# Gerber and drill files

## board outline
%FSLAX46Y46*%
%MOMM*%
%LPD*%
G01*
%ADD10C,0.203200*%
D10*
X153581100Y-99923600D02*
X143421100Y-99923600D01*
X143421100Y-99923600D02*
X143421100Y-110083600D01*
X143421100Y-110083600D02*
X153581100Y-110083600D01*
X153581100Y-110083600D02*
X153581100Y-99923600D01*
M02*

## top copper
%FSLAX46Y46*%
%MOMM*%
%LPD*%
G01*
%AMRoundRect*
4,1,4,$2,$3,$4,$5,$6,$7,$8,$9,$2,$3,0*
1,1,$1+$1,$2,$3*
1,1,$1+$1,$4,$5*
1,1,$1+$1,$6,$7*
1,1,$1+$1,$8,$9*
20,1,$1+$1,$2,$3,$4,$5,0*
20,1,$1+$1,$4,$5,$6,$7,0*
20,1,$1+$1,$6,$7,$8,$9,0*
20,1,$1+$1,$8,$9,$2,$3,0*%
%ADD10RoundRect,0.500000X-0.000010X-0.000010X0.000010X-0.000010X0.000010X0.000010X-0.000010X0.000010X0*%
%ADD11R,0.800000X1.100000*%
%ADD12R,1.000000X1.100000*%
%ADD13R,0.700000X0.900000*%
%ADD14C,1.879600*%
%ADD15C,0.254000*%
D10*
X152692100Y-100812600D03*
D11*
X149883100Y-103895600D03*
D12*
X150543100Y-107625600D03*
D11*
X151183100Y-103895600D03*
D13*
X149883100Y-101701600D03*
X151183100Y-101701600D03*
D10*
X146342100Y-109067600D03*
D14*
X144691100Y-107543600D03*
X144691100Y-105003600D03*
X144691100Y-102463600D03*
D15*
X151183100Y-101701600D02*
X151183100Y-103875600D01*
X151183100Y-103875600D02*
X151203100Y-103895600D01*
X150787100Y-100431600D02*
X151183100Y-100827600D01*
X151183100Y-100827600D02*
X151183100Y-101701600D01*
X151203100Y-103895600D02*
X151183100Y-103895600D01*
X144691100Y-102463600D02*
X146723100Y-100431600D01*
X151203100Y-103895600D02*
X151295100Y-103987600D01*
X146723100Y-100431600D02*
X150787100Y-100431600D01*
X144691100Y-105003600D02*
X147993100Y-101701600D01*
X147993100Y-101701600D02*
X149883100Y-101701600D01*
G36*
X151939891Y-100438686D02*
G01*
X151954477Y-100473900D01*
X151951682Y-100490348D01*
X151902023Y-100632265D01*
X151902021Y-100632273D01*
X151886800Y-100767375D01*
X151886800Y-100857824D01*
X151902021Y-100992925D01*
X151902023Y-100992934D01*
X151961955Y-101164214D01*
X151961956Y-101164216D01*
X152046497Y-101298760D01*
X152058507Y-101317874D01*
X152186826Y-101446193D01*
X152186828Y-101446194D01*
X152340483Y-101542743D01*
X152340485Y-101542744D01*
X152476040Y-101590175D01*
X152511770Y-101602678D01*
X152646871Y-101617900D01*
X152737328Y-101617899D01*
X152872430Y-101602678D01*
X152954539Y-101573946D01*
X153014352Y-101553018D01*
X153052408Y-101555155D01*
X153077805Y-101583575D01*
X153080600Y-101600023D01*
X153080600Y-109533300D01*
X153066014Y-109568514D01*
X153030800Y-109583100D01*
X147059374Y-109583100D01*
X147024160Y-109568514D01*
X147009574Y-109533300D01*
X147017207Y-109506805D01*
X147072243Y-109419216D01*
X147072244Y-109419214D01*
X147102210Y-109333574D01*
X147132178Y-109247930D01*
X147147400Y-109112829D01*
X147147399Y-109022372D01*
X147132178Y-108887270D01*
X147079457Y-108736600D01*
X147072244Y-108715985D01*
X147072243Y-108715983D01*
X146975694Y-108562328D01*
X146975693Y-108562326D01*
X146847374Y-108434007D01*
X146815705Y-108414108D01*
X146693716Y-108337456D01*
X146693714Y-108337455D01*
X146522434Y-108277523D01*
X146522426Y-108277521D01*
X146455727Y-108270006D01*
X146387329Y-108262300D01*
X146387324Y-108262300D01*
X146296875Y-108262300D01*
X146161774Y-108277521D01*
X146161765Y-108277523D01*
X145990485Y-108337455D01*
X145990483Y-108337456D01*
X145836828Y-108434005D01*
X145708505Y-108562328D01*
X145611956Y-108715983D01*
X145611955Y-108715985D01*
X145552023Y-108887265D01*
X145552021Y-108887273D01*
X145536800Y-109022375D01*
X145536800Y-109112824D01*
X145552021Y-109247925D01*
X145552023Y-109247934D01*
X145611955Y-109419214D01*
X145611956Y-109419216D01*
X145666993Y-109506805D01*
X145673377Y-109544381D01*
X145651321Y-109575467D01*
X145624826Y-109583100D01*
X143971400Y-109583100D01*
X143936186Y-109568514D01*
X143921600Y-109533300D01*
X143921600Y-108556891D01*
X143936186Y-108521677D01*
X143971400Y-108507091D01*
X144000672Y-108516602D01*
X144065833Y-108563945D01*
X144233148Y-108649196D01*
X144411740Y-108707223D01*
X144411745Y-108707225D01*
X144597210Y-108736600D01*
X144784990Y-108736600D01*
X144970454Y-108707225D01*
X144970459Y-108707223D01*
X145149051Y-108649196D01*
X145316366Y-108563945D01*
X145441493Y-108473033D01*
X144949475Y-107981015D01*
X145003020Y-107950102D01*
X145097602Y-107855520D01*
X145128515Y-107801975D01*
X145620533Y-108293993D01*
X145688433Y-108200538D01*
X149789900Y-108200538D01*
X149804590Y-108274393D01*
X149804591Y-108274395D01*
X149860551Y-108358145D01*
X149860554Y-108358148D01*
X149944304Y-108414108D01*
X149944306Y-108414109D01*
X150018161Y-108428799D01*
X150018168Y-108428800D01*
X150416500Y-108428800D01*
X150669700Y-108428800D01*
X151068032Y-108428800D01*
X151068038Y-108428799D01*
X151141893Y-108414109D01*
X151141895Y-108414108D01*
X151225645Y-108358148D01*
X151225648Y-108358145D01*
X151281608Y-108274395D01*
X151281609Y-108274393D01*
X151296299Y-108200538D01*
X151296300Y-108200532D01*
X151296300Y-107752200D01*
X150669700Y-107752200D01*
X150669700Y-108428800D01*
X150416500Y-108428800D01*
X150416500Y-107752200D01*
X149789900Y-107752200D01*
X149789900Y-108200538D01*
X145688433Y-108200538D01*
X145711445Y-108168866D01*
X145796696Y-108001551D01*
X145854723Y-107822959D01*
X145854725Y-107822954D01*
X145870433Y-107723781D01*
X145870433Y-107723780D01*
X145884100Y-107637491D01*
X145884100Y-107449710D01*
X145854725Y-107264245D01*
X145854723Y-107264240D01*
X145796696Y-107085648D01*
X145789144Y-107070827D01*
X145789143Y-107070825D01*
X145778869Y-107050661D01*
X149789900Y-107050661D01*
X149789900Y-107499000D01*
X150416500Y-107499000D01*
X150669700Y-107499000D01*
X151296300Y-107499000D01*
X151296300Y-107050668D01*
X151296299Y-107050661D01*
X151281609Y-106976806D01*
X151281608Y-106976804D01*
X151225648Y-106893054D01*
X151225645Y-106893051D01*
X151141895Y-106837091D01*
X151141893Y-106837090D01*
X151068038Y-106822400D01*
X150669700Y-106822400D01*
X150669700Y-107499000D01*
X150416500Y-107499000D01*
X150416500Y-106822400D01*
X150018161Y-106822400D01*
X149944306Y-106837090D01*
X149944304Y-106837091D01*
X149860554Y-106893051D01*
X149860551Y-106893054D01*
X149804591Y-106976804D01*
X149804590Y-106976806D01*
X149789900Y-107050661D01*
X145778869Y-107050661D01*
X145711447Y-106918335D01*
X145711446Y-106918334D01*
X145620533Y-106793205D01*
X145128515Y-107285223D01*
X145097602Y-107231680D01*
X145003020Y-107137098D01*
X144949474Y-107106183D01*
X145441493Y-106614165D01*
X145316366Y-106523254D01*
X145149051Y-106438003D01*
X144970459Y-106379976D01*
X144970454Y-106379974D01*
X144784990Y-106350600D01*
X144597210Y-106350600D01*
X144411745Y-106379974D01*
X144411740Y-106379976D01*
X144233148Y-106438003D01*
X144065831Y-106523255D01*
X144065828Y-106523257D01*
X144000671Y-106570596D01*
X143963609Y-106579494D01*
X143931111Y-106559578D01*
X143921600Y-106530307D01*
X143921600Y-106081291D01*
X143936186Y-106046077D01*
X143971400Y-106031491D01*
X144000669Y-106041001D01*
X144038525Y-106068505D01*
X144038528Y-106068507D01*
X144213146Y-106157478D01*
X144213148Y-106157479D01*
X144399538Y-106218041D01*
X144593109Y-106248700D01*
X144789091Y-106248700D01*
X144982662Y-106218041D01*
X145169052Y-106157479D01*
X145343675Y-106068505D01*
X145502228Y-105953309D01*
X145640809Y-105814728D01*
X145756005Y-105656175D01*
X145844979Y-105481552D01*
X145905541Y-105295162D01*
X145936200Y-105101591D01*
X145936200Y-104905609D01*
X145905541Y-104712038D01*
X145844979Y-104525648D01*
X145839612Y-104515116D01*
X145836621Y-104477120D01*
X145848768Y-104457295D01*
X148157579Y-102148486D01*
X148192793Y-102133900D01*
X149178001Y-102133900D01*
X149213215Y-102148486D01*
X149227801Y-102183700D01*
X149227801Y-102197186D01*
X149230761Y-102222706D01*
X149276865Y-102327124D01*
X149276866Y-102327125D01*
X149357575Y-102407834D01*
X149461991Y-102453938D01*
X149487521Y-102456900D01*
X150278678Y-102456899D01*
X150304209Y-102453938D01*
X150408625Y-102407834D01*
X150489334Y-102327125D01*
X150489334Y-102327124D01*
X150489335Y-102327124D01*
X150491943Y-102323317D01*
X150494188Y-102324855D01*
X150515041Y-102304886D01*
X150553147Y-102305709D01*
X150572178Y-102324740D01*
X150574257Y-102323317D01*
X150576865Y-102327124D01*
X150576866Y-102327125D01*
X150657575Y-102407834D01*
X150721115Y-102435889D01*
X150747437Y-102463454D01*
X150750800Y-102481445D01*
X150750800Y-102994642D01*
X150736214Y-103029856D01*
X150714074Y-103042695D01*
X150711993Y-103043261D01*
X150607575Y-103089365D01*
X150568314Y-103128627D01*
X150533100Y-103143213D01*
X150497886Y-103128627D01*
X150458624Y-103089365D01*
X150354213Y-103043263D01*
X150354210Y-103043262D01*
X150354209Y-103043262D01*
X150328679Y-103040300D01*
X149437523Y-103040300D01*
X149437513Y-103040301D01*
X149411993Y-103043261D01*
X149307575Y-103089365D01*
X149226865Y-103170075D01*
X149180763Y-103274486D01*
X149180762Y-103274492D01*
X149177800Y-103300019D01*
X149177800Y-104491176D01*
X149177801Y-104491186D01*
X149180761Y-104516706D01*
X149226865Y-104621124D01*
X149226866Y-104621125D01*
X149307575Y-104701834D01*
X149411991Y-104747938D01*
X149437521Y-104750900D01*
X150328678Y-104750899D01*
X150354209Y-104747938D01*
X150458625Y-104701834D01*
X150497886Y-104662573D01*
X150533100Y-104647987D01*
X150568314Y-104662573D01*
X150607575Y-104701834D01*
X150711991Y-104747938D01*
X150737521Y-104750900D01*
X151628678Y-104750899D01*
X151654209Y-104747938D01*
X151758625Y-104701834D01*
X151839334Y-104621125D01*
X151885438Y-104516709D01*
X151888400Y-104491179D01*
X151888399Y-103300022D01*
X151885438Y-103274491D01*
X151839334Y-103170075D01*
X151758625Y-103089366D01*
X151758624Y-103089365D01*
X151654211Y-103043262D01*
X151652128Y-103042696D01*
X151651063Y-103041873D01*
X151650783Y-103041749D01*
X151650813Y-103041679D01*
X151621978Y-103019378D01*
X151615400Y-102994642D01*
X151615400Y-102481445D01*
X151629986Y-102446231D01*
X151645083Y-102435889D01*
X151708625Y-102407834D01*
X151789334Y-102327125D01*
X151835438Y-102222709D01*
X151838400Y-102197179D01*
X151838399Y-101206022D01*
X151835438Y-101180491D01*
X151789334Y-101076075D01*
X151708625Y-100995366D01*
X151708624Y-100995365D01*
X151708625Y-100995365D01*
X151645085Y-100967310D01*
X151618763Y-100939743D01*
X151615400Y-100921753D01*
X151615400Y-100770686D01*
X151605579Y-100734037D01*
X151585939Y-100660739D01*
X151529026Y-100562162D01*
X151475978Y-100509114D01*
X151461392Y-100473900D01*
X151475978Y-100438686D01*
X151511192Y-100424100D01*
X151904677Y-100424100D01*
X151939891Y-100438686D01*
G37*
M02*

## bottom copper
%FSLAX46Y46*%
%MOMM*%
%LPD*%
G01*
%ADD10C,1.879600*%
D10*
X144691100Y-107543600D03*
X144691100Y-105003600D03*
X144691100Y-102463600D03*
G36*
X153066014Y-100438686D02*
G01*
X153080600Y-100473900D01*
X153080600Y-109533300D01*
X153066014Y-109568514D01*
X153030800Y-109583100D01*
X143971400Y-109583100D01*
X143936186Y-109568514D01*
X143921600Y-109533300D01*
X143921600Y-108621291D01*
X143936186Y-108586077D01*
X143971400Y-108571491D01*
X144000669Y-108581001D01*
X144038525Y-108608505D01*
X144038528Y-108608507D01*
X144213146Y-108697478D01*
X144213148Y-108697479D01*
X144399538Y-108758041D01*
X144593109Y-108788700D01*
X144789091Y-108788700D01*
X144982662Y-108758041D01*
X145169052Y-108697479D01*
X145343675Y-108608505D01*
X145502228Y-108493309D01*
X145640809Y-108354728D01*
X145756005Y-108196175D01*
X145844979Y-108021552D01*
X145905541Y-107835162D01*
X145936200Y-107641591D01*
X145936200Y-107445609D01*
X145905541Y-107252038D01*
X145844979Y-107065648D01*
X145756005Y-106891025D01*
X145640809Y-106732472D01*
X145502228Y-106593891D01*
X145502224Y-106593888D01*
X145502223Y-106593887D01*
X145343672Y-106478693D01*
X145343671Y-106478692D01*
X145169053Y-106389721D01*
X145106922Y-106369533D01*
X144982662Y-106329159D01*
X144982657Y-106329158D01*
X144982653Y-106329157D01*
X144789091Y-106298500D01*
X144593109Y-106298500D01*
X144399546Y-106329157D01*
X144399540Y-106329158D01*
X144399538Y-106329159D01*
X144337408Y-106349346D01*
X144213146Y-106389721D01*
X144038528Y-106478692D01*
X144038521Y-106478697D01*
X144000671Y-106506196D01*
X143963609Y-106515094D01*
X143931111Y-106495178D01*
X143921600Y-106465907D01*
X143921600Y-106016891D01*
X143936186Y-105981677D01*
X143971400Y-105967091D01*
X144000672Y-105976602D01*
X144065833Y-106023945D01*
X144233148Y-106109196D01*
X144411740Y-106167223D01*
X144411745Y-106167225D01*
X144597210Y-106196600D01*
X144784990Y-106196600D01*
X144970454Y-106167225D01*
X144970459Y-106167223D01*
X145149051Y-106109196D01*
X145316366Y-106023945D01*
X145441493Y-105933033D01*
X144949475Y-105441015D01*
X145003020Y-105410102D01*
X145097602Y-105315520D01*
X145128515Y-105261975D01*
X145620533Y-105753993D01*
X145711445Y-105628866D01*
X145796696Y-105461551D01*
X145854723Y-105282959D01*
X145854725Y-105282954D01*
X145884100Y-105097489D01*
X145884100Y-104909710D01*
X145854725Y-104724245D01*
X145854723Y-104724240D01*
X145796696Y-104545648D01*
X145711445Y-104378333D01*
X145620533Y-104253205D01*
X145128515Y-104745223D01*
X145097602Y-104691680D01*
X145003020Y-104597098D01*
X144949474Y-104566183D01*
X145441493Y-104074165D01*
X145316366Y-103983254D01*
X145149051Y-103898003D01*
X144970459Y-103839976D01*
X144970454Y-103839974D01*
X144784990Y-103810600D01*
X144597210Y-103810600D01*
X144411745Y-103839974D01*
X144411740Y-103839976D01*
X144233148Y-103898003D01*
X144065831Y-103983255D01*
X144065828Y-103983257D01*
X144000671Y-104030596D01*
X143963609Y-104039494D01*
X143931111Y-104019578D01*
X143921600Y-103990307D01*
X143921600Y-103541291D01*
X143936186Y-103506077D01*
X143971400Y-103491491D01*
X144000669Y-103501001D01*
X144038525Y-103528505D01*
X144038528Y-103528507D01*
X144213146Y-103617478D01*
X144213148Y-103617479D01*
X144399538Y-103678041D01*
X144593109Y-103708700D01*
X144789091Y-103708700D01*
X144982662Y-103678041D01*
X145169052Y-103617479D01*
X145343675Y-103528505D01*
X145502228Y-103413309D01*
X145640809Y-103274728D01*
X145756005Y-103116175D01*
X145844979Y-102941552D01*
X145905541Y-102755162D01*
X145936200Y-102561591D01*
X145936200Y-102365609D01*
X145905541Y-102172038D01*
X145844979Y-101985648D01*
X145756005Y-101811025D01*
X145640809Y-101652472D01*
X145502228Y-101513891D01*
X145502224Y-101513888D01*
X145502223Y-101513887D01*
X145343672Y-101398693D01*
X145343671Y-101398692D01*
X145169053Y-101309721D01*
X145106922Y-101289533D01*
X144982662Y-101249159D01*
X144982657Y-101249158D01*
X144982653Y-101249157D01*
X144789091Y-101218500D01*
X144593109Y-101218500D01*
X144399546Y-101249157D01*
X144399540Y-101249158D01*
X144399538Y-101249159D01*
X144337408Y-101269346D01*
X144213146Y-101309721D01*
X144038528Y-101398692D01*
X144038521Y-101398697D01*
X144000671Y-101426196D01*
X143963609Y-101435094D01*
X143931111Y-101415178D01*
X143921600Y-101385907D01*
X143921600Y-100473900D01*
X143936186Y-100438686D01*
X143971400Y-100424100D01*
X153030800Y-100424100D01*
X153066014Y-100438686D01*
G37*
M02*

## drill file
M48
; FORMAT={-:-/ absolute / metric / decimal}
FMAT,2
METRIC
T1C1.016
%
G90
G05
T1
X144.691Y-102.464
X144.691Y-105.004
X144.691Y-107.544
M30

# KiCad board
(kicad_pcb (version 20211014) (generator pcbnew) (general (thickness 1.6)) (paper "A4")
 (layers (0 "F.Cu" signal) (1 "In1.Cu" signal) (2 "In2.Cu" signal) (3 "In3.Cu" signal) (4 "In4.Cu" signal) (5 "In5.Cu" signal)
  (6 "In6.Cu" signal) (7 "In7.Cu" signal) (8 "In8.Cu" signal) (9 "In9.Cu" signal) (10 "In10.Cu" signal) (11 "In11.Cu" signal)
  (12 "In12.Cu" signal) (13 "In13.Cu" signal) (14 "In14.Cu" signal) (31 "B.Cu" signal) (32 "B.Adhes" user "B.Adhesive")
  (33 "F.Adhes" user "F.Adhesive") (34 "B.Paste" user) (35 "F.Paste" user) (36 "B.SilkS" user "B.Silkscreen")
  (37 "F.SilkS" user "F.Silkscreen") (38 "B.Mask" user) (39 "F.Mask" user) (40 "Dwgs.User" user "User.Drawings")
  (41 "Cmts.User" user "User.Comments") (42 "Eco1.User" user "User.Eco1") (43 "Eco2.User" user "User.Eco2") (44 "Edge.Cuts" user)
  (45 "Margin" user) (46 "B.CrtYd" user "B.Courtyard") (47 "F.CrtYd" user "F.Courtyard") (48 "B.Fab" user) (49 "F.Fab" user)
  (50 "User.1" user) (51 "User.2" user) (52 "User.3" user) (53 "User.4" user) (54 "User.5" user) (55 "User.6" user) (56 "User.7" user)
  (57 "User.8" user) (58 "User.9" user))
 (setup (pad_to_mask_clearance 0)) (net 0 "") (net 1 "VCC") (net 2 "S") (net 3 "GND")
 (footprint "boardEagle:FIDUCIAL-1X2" (layer "F.Cu") (at 152.6921 100.8126)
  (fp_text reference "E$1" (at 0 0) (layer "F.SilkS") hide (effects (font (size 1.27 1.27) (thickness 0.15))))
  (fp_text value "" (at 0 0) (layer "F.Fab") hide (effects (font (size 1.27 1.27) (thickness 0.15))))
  (pad "1" smd roundrect (at 0 0) (size 1 1) (layers "F.Cu" "F.Mask") (roundrect_rratio 0.5) (solder_mask_margin 0.1016)))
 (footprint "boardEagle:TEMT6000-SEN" (layer "F.Cu") (at 150.5331 105.7656 -90)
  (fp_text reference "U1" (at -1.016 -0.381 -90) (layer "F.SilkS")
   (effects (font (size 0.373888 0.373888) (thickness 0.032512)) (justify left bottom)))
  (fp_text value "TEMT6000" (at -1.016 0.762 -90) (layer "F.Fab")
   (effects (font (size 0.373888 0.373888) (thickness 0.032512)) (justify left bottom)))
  (pad "BASE" smd rect (at -1.87 0.65 270) (size 1.1 0.8) (layers "F.Cu" "F.Paste" "F.Mask") (solder_mask_margin 0.1016))
  (pad "COLLECTOR" smd rect (at 1.86 -0.01 270) (size 1.1 1) (layers "F.Cu" "F.Paste" "F.Mask") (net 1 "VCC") (solder_mask_margin 0.1016))
  (pad "EMITTER" smd rect (at -1.87 -0.65 270) (size 1.1 0.8) (layers "F.Cu" "F.Paste" "F.Mask") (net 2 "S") (solder_mask_margin 0.1016)))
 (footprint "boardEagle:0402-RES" (layer "F.Cu") (at 150.5331 101.7016)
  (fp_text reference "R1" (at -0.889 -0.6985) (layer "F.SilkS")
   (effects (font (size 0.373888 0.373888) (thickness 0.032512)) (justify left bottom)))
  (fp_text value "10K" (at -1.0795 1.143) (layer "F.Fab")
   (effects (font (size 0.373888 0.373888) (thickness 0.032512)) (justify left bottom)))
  (pad "1" smd rect (at -0.65 0) (size 0.7 0.9) (layers "F.Cu" "F.Paste" "F.Mask") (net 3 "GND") (solder_mask_margin 0.1016))
  (pad "2" smd rect (at 0.65 0) (size 0.7 0.9) (layers "F.Cu" "F.Paste" "F.Mask") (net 2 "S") (solder_mask_margin 0.1016)))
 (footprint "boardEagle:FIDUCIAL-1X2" (layer "F.Cu") (at 146.3421 109.0676)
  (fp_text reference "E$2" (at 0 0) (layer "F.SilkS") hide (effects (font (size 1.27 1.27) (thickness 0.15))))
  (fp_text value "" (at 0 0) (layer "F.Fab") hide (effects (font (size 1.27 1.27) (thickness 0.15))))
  (pad "1" smd roundrect (at 0 0) (size 1 1) (layers "F.Cu" "F.Mask") (roundrect_rratio 0.5) (solder_mask_margin 0.1016)))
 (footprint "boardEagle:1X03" (layer "F.Cu") (at 144.6911 107.5436 90)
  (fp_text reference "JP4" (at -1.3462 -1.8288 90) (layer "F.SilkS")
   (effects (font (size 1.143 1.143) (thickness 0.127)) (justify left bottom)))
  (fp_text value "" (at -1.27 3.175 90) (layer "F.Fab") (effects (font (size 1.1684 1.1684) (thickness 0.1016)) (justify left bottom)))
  (pad "1" thru_hole circle (at 0 0 180) (size 1.8796 1.8796) (drill 1.016) (layers *.Cu *.Mask) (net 1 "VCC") (solder_mask_margin 0.1016))
  (pad "2" thru_hole circle (at 2.54 0 180) (size 1.8796 1.8796) (drill 1.016) (layers *.Cu *.Mask) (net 3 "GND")
   (solder_mask_margin 0.1016))
  (pad "3" thru_hole circle (at 5.08 0 180) (size 1.8796 1.8796) (drill 1.016) (layers *.Cu *.Mask) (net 2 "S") (solder_mask_margin 0.1016)))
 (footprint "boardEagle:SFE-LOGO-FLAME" (layer "B.Cu") (at 149.5171 106.5276 180)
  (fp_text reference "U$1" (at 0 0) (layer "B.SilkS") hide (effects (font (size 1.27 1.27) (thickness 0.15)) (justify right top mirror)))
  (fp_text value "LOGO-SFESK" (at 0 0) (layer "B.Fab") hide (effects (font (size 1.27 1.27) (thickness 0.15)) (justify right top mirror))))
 (gr_line (start 153.5811 99.9236) (end 143.4211 99.9236) (layer "Edge.Cuts") (width 0.2032))
 (gr_line (start 143.4211 99.9236) (end 143.4211 110.0836) (layer "Edge.Cuts") (width 0.2032))
 (gr_line (start 143.4211 110.0836) (end 153.5811 110.0836) (layer "Edge.Cuts") (width 0.2032))
 (gr_line (start 153.5811 110.0836) (end 153.5811 99.9236) (layer "Edge.Cuts") (width 0.2032))
 (segment (start 151.1831 101.7016) (end 151.1831 103.8756) (width 0.254) (layer "F.Cu") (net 2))
 (segment (start 151.1831 103.8756) (end 151.2031 103.8956) (width 0.254) (layer "F.Cu") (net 2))
 (segment (start 150.7871 100.4316) (end 151.1831 100.8276) (width 0.254) (layer "F.Cu") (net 2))
 (segment (start 151.1831 100.8276) (end 151.1831 101.7016) (width 0.254) (layer "F.Cu") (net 2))
 (segment (start 151.2031 103.8956) (end 151.1831 103.8956) (width 0.254) (layer "F.Cu") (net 2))
 (segment (start 144.6911 102.4636) (end 146.7231 100.4316) (width 0.254) (layer "F.Cu") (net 2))
 (segment (start 151.2031 103.8956) (end 151.2951 103.9876) (width 0.254) (layer "F.Cu") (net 2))
 (segment (start 146.7231 100.4316) (end 150.7871 100.4316) (width 0.254) (layer "F.Cu") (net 2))
 (segment (start 144.6911 105.0036) (end 147.9931 101.7016) (width 0.254) (layer "F.Cu") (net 3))
 (segment (start 147.9931 101.7016) (end 149.8831 101.7016) (width 0.254) (layer "F.Cu") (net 3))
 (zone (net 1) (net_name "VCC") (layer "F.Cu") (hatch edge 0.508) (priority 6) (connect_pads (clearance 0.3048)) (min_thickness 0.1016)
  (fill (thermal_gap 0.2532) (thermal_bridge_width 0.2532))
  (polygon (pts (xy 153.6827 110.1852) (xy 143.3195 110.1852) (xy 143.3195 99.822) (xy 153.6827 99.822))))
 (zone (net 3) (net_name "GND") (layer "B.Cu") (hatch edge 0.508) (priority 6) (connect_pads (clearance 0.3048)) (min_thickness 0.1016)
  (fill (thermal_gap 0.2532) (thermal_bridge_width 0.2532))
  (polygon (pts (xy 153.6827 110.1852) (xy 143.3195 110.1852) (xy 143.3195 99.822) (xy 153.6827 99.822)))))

